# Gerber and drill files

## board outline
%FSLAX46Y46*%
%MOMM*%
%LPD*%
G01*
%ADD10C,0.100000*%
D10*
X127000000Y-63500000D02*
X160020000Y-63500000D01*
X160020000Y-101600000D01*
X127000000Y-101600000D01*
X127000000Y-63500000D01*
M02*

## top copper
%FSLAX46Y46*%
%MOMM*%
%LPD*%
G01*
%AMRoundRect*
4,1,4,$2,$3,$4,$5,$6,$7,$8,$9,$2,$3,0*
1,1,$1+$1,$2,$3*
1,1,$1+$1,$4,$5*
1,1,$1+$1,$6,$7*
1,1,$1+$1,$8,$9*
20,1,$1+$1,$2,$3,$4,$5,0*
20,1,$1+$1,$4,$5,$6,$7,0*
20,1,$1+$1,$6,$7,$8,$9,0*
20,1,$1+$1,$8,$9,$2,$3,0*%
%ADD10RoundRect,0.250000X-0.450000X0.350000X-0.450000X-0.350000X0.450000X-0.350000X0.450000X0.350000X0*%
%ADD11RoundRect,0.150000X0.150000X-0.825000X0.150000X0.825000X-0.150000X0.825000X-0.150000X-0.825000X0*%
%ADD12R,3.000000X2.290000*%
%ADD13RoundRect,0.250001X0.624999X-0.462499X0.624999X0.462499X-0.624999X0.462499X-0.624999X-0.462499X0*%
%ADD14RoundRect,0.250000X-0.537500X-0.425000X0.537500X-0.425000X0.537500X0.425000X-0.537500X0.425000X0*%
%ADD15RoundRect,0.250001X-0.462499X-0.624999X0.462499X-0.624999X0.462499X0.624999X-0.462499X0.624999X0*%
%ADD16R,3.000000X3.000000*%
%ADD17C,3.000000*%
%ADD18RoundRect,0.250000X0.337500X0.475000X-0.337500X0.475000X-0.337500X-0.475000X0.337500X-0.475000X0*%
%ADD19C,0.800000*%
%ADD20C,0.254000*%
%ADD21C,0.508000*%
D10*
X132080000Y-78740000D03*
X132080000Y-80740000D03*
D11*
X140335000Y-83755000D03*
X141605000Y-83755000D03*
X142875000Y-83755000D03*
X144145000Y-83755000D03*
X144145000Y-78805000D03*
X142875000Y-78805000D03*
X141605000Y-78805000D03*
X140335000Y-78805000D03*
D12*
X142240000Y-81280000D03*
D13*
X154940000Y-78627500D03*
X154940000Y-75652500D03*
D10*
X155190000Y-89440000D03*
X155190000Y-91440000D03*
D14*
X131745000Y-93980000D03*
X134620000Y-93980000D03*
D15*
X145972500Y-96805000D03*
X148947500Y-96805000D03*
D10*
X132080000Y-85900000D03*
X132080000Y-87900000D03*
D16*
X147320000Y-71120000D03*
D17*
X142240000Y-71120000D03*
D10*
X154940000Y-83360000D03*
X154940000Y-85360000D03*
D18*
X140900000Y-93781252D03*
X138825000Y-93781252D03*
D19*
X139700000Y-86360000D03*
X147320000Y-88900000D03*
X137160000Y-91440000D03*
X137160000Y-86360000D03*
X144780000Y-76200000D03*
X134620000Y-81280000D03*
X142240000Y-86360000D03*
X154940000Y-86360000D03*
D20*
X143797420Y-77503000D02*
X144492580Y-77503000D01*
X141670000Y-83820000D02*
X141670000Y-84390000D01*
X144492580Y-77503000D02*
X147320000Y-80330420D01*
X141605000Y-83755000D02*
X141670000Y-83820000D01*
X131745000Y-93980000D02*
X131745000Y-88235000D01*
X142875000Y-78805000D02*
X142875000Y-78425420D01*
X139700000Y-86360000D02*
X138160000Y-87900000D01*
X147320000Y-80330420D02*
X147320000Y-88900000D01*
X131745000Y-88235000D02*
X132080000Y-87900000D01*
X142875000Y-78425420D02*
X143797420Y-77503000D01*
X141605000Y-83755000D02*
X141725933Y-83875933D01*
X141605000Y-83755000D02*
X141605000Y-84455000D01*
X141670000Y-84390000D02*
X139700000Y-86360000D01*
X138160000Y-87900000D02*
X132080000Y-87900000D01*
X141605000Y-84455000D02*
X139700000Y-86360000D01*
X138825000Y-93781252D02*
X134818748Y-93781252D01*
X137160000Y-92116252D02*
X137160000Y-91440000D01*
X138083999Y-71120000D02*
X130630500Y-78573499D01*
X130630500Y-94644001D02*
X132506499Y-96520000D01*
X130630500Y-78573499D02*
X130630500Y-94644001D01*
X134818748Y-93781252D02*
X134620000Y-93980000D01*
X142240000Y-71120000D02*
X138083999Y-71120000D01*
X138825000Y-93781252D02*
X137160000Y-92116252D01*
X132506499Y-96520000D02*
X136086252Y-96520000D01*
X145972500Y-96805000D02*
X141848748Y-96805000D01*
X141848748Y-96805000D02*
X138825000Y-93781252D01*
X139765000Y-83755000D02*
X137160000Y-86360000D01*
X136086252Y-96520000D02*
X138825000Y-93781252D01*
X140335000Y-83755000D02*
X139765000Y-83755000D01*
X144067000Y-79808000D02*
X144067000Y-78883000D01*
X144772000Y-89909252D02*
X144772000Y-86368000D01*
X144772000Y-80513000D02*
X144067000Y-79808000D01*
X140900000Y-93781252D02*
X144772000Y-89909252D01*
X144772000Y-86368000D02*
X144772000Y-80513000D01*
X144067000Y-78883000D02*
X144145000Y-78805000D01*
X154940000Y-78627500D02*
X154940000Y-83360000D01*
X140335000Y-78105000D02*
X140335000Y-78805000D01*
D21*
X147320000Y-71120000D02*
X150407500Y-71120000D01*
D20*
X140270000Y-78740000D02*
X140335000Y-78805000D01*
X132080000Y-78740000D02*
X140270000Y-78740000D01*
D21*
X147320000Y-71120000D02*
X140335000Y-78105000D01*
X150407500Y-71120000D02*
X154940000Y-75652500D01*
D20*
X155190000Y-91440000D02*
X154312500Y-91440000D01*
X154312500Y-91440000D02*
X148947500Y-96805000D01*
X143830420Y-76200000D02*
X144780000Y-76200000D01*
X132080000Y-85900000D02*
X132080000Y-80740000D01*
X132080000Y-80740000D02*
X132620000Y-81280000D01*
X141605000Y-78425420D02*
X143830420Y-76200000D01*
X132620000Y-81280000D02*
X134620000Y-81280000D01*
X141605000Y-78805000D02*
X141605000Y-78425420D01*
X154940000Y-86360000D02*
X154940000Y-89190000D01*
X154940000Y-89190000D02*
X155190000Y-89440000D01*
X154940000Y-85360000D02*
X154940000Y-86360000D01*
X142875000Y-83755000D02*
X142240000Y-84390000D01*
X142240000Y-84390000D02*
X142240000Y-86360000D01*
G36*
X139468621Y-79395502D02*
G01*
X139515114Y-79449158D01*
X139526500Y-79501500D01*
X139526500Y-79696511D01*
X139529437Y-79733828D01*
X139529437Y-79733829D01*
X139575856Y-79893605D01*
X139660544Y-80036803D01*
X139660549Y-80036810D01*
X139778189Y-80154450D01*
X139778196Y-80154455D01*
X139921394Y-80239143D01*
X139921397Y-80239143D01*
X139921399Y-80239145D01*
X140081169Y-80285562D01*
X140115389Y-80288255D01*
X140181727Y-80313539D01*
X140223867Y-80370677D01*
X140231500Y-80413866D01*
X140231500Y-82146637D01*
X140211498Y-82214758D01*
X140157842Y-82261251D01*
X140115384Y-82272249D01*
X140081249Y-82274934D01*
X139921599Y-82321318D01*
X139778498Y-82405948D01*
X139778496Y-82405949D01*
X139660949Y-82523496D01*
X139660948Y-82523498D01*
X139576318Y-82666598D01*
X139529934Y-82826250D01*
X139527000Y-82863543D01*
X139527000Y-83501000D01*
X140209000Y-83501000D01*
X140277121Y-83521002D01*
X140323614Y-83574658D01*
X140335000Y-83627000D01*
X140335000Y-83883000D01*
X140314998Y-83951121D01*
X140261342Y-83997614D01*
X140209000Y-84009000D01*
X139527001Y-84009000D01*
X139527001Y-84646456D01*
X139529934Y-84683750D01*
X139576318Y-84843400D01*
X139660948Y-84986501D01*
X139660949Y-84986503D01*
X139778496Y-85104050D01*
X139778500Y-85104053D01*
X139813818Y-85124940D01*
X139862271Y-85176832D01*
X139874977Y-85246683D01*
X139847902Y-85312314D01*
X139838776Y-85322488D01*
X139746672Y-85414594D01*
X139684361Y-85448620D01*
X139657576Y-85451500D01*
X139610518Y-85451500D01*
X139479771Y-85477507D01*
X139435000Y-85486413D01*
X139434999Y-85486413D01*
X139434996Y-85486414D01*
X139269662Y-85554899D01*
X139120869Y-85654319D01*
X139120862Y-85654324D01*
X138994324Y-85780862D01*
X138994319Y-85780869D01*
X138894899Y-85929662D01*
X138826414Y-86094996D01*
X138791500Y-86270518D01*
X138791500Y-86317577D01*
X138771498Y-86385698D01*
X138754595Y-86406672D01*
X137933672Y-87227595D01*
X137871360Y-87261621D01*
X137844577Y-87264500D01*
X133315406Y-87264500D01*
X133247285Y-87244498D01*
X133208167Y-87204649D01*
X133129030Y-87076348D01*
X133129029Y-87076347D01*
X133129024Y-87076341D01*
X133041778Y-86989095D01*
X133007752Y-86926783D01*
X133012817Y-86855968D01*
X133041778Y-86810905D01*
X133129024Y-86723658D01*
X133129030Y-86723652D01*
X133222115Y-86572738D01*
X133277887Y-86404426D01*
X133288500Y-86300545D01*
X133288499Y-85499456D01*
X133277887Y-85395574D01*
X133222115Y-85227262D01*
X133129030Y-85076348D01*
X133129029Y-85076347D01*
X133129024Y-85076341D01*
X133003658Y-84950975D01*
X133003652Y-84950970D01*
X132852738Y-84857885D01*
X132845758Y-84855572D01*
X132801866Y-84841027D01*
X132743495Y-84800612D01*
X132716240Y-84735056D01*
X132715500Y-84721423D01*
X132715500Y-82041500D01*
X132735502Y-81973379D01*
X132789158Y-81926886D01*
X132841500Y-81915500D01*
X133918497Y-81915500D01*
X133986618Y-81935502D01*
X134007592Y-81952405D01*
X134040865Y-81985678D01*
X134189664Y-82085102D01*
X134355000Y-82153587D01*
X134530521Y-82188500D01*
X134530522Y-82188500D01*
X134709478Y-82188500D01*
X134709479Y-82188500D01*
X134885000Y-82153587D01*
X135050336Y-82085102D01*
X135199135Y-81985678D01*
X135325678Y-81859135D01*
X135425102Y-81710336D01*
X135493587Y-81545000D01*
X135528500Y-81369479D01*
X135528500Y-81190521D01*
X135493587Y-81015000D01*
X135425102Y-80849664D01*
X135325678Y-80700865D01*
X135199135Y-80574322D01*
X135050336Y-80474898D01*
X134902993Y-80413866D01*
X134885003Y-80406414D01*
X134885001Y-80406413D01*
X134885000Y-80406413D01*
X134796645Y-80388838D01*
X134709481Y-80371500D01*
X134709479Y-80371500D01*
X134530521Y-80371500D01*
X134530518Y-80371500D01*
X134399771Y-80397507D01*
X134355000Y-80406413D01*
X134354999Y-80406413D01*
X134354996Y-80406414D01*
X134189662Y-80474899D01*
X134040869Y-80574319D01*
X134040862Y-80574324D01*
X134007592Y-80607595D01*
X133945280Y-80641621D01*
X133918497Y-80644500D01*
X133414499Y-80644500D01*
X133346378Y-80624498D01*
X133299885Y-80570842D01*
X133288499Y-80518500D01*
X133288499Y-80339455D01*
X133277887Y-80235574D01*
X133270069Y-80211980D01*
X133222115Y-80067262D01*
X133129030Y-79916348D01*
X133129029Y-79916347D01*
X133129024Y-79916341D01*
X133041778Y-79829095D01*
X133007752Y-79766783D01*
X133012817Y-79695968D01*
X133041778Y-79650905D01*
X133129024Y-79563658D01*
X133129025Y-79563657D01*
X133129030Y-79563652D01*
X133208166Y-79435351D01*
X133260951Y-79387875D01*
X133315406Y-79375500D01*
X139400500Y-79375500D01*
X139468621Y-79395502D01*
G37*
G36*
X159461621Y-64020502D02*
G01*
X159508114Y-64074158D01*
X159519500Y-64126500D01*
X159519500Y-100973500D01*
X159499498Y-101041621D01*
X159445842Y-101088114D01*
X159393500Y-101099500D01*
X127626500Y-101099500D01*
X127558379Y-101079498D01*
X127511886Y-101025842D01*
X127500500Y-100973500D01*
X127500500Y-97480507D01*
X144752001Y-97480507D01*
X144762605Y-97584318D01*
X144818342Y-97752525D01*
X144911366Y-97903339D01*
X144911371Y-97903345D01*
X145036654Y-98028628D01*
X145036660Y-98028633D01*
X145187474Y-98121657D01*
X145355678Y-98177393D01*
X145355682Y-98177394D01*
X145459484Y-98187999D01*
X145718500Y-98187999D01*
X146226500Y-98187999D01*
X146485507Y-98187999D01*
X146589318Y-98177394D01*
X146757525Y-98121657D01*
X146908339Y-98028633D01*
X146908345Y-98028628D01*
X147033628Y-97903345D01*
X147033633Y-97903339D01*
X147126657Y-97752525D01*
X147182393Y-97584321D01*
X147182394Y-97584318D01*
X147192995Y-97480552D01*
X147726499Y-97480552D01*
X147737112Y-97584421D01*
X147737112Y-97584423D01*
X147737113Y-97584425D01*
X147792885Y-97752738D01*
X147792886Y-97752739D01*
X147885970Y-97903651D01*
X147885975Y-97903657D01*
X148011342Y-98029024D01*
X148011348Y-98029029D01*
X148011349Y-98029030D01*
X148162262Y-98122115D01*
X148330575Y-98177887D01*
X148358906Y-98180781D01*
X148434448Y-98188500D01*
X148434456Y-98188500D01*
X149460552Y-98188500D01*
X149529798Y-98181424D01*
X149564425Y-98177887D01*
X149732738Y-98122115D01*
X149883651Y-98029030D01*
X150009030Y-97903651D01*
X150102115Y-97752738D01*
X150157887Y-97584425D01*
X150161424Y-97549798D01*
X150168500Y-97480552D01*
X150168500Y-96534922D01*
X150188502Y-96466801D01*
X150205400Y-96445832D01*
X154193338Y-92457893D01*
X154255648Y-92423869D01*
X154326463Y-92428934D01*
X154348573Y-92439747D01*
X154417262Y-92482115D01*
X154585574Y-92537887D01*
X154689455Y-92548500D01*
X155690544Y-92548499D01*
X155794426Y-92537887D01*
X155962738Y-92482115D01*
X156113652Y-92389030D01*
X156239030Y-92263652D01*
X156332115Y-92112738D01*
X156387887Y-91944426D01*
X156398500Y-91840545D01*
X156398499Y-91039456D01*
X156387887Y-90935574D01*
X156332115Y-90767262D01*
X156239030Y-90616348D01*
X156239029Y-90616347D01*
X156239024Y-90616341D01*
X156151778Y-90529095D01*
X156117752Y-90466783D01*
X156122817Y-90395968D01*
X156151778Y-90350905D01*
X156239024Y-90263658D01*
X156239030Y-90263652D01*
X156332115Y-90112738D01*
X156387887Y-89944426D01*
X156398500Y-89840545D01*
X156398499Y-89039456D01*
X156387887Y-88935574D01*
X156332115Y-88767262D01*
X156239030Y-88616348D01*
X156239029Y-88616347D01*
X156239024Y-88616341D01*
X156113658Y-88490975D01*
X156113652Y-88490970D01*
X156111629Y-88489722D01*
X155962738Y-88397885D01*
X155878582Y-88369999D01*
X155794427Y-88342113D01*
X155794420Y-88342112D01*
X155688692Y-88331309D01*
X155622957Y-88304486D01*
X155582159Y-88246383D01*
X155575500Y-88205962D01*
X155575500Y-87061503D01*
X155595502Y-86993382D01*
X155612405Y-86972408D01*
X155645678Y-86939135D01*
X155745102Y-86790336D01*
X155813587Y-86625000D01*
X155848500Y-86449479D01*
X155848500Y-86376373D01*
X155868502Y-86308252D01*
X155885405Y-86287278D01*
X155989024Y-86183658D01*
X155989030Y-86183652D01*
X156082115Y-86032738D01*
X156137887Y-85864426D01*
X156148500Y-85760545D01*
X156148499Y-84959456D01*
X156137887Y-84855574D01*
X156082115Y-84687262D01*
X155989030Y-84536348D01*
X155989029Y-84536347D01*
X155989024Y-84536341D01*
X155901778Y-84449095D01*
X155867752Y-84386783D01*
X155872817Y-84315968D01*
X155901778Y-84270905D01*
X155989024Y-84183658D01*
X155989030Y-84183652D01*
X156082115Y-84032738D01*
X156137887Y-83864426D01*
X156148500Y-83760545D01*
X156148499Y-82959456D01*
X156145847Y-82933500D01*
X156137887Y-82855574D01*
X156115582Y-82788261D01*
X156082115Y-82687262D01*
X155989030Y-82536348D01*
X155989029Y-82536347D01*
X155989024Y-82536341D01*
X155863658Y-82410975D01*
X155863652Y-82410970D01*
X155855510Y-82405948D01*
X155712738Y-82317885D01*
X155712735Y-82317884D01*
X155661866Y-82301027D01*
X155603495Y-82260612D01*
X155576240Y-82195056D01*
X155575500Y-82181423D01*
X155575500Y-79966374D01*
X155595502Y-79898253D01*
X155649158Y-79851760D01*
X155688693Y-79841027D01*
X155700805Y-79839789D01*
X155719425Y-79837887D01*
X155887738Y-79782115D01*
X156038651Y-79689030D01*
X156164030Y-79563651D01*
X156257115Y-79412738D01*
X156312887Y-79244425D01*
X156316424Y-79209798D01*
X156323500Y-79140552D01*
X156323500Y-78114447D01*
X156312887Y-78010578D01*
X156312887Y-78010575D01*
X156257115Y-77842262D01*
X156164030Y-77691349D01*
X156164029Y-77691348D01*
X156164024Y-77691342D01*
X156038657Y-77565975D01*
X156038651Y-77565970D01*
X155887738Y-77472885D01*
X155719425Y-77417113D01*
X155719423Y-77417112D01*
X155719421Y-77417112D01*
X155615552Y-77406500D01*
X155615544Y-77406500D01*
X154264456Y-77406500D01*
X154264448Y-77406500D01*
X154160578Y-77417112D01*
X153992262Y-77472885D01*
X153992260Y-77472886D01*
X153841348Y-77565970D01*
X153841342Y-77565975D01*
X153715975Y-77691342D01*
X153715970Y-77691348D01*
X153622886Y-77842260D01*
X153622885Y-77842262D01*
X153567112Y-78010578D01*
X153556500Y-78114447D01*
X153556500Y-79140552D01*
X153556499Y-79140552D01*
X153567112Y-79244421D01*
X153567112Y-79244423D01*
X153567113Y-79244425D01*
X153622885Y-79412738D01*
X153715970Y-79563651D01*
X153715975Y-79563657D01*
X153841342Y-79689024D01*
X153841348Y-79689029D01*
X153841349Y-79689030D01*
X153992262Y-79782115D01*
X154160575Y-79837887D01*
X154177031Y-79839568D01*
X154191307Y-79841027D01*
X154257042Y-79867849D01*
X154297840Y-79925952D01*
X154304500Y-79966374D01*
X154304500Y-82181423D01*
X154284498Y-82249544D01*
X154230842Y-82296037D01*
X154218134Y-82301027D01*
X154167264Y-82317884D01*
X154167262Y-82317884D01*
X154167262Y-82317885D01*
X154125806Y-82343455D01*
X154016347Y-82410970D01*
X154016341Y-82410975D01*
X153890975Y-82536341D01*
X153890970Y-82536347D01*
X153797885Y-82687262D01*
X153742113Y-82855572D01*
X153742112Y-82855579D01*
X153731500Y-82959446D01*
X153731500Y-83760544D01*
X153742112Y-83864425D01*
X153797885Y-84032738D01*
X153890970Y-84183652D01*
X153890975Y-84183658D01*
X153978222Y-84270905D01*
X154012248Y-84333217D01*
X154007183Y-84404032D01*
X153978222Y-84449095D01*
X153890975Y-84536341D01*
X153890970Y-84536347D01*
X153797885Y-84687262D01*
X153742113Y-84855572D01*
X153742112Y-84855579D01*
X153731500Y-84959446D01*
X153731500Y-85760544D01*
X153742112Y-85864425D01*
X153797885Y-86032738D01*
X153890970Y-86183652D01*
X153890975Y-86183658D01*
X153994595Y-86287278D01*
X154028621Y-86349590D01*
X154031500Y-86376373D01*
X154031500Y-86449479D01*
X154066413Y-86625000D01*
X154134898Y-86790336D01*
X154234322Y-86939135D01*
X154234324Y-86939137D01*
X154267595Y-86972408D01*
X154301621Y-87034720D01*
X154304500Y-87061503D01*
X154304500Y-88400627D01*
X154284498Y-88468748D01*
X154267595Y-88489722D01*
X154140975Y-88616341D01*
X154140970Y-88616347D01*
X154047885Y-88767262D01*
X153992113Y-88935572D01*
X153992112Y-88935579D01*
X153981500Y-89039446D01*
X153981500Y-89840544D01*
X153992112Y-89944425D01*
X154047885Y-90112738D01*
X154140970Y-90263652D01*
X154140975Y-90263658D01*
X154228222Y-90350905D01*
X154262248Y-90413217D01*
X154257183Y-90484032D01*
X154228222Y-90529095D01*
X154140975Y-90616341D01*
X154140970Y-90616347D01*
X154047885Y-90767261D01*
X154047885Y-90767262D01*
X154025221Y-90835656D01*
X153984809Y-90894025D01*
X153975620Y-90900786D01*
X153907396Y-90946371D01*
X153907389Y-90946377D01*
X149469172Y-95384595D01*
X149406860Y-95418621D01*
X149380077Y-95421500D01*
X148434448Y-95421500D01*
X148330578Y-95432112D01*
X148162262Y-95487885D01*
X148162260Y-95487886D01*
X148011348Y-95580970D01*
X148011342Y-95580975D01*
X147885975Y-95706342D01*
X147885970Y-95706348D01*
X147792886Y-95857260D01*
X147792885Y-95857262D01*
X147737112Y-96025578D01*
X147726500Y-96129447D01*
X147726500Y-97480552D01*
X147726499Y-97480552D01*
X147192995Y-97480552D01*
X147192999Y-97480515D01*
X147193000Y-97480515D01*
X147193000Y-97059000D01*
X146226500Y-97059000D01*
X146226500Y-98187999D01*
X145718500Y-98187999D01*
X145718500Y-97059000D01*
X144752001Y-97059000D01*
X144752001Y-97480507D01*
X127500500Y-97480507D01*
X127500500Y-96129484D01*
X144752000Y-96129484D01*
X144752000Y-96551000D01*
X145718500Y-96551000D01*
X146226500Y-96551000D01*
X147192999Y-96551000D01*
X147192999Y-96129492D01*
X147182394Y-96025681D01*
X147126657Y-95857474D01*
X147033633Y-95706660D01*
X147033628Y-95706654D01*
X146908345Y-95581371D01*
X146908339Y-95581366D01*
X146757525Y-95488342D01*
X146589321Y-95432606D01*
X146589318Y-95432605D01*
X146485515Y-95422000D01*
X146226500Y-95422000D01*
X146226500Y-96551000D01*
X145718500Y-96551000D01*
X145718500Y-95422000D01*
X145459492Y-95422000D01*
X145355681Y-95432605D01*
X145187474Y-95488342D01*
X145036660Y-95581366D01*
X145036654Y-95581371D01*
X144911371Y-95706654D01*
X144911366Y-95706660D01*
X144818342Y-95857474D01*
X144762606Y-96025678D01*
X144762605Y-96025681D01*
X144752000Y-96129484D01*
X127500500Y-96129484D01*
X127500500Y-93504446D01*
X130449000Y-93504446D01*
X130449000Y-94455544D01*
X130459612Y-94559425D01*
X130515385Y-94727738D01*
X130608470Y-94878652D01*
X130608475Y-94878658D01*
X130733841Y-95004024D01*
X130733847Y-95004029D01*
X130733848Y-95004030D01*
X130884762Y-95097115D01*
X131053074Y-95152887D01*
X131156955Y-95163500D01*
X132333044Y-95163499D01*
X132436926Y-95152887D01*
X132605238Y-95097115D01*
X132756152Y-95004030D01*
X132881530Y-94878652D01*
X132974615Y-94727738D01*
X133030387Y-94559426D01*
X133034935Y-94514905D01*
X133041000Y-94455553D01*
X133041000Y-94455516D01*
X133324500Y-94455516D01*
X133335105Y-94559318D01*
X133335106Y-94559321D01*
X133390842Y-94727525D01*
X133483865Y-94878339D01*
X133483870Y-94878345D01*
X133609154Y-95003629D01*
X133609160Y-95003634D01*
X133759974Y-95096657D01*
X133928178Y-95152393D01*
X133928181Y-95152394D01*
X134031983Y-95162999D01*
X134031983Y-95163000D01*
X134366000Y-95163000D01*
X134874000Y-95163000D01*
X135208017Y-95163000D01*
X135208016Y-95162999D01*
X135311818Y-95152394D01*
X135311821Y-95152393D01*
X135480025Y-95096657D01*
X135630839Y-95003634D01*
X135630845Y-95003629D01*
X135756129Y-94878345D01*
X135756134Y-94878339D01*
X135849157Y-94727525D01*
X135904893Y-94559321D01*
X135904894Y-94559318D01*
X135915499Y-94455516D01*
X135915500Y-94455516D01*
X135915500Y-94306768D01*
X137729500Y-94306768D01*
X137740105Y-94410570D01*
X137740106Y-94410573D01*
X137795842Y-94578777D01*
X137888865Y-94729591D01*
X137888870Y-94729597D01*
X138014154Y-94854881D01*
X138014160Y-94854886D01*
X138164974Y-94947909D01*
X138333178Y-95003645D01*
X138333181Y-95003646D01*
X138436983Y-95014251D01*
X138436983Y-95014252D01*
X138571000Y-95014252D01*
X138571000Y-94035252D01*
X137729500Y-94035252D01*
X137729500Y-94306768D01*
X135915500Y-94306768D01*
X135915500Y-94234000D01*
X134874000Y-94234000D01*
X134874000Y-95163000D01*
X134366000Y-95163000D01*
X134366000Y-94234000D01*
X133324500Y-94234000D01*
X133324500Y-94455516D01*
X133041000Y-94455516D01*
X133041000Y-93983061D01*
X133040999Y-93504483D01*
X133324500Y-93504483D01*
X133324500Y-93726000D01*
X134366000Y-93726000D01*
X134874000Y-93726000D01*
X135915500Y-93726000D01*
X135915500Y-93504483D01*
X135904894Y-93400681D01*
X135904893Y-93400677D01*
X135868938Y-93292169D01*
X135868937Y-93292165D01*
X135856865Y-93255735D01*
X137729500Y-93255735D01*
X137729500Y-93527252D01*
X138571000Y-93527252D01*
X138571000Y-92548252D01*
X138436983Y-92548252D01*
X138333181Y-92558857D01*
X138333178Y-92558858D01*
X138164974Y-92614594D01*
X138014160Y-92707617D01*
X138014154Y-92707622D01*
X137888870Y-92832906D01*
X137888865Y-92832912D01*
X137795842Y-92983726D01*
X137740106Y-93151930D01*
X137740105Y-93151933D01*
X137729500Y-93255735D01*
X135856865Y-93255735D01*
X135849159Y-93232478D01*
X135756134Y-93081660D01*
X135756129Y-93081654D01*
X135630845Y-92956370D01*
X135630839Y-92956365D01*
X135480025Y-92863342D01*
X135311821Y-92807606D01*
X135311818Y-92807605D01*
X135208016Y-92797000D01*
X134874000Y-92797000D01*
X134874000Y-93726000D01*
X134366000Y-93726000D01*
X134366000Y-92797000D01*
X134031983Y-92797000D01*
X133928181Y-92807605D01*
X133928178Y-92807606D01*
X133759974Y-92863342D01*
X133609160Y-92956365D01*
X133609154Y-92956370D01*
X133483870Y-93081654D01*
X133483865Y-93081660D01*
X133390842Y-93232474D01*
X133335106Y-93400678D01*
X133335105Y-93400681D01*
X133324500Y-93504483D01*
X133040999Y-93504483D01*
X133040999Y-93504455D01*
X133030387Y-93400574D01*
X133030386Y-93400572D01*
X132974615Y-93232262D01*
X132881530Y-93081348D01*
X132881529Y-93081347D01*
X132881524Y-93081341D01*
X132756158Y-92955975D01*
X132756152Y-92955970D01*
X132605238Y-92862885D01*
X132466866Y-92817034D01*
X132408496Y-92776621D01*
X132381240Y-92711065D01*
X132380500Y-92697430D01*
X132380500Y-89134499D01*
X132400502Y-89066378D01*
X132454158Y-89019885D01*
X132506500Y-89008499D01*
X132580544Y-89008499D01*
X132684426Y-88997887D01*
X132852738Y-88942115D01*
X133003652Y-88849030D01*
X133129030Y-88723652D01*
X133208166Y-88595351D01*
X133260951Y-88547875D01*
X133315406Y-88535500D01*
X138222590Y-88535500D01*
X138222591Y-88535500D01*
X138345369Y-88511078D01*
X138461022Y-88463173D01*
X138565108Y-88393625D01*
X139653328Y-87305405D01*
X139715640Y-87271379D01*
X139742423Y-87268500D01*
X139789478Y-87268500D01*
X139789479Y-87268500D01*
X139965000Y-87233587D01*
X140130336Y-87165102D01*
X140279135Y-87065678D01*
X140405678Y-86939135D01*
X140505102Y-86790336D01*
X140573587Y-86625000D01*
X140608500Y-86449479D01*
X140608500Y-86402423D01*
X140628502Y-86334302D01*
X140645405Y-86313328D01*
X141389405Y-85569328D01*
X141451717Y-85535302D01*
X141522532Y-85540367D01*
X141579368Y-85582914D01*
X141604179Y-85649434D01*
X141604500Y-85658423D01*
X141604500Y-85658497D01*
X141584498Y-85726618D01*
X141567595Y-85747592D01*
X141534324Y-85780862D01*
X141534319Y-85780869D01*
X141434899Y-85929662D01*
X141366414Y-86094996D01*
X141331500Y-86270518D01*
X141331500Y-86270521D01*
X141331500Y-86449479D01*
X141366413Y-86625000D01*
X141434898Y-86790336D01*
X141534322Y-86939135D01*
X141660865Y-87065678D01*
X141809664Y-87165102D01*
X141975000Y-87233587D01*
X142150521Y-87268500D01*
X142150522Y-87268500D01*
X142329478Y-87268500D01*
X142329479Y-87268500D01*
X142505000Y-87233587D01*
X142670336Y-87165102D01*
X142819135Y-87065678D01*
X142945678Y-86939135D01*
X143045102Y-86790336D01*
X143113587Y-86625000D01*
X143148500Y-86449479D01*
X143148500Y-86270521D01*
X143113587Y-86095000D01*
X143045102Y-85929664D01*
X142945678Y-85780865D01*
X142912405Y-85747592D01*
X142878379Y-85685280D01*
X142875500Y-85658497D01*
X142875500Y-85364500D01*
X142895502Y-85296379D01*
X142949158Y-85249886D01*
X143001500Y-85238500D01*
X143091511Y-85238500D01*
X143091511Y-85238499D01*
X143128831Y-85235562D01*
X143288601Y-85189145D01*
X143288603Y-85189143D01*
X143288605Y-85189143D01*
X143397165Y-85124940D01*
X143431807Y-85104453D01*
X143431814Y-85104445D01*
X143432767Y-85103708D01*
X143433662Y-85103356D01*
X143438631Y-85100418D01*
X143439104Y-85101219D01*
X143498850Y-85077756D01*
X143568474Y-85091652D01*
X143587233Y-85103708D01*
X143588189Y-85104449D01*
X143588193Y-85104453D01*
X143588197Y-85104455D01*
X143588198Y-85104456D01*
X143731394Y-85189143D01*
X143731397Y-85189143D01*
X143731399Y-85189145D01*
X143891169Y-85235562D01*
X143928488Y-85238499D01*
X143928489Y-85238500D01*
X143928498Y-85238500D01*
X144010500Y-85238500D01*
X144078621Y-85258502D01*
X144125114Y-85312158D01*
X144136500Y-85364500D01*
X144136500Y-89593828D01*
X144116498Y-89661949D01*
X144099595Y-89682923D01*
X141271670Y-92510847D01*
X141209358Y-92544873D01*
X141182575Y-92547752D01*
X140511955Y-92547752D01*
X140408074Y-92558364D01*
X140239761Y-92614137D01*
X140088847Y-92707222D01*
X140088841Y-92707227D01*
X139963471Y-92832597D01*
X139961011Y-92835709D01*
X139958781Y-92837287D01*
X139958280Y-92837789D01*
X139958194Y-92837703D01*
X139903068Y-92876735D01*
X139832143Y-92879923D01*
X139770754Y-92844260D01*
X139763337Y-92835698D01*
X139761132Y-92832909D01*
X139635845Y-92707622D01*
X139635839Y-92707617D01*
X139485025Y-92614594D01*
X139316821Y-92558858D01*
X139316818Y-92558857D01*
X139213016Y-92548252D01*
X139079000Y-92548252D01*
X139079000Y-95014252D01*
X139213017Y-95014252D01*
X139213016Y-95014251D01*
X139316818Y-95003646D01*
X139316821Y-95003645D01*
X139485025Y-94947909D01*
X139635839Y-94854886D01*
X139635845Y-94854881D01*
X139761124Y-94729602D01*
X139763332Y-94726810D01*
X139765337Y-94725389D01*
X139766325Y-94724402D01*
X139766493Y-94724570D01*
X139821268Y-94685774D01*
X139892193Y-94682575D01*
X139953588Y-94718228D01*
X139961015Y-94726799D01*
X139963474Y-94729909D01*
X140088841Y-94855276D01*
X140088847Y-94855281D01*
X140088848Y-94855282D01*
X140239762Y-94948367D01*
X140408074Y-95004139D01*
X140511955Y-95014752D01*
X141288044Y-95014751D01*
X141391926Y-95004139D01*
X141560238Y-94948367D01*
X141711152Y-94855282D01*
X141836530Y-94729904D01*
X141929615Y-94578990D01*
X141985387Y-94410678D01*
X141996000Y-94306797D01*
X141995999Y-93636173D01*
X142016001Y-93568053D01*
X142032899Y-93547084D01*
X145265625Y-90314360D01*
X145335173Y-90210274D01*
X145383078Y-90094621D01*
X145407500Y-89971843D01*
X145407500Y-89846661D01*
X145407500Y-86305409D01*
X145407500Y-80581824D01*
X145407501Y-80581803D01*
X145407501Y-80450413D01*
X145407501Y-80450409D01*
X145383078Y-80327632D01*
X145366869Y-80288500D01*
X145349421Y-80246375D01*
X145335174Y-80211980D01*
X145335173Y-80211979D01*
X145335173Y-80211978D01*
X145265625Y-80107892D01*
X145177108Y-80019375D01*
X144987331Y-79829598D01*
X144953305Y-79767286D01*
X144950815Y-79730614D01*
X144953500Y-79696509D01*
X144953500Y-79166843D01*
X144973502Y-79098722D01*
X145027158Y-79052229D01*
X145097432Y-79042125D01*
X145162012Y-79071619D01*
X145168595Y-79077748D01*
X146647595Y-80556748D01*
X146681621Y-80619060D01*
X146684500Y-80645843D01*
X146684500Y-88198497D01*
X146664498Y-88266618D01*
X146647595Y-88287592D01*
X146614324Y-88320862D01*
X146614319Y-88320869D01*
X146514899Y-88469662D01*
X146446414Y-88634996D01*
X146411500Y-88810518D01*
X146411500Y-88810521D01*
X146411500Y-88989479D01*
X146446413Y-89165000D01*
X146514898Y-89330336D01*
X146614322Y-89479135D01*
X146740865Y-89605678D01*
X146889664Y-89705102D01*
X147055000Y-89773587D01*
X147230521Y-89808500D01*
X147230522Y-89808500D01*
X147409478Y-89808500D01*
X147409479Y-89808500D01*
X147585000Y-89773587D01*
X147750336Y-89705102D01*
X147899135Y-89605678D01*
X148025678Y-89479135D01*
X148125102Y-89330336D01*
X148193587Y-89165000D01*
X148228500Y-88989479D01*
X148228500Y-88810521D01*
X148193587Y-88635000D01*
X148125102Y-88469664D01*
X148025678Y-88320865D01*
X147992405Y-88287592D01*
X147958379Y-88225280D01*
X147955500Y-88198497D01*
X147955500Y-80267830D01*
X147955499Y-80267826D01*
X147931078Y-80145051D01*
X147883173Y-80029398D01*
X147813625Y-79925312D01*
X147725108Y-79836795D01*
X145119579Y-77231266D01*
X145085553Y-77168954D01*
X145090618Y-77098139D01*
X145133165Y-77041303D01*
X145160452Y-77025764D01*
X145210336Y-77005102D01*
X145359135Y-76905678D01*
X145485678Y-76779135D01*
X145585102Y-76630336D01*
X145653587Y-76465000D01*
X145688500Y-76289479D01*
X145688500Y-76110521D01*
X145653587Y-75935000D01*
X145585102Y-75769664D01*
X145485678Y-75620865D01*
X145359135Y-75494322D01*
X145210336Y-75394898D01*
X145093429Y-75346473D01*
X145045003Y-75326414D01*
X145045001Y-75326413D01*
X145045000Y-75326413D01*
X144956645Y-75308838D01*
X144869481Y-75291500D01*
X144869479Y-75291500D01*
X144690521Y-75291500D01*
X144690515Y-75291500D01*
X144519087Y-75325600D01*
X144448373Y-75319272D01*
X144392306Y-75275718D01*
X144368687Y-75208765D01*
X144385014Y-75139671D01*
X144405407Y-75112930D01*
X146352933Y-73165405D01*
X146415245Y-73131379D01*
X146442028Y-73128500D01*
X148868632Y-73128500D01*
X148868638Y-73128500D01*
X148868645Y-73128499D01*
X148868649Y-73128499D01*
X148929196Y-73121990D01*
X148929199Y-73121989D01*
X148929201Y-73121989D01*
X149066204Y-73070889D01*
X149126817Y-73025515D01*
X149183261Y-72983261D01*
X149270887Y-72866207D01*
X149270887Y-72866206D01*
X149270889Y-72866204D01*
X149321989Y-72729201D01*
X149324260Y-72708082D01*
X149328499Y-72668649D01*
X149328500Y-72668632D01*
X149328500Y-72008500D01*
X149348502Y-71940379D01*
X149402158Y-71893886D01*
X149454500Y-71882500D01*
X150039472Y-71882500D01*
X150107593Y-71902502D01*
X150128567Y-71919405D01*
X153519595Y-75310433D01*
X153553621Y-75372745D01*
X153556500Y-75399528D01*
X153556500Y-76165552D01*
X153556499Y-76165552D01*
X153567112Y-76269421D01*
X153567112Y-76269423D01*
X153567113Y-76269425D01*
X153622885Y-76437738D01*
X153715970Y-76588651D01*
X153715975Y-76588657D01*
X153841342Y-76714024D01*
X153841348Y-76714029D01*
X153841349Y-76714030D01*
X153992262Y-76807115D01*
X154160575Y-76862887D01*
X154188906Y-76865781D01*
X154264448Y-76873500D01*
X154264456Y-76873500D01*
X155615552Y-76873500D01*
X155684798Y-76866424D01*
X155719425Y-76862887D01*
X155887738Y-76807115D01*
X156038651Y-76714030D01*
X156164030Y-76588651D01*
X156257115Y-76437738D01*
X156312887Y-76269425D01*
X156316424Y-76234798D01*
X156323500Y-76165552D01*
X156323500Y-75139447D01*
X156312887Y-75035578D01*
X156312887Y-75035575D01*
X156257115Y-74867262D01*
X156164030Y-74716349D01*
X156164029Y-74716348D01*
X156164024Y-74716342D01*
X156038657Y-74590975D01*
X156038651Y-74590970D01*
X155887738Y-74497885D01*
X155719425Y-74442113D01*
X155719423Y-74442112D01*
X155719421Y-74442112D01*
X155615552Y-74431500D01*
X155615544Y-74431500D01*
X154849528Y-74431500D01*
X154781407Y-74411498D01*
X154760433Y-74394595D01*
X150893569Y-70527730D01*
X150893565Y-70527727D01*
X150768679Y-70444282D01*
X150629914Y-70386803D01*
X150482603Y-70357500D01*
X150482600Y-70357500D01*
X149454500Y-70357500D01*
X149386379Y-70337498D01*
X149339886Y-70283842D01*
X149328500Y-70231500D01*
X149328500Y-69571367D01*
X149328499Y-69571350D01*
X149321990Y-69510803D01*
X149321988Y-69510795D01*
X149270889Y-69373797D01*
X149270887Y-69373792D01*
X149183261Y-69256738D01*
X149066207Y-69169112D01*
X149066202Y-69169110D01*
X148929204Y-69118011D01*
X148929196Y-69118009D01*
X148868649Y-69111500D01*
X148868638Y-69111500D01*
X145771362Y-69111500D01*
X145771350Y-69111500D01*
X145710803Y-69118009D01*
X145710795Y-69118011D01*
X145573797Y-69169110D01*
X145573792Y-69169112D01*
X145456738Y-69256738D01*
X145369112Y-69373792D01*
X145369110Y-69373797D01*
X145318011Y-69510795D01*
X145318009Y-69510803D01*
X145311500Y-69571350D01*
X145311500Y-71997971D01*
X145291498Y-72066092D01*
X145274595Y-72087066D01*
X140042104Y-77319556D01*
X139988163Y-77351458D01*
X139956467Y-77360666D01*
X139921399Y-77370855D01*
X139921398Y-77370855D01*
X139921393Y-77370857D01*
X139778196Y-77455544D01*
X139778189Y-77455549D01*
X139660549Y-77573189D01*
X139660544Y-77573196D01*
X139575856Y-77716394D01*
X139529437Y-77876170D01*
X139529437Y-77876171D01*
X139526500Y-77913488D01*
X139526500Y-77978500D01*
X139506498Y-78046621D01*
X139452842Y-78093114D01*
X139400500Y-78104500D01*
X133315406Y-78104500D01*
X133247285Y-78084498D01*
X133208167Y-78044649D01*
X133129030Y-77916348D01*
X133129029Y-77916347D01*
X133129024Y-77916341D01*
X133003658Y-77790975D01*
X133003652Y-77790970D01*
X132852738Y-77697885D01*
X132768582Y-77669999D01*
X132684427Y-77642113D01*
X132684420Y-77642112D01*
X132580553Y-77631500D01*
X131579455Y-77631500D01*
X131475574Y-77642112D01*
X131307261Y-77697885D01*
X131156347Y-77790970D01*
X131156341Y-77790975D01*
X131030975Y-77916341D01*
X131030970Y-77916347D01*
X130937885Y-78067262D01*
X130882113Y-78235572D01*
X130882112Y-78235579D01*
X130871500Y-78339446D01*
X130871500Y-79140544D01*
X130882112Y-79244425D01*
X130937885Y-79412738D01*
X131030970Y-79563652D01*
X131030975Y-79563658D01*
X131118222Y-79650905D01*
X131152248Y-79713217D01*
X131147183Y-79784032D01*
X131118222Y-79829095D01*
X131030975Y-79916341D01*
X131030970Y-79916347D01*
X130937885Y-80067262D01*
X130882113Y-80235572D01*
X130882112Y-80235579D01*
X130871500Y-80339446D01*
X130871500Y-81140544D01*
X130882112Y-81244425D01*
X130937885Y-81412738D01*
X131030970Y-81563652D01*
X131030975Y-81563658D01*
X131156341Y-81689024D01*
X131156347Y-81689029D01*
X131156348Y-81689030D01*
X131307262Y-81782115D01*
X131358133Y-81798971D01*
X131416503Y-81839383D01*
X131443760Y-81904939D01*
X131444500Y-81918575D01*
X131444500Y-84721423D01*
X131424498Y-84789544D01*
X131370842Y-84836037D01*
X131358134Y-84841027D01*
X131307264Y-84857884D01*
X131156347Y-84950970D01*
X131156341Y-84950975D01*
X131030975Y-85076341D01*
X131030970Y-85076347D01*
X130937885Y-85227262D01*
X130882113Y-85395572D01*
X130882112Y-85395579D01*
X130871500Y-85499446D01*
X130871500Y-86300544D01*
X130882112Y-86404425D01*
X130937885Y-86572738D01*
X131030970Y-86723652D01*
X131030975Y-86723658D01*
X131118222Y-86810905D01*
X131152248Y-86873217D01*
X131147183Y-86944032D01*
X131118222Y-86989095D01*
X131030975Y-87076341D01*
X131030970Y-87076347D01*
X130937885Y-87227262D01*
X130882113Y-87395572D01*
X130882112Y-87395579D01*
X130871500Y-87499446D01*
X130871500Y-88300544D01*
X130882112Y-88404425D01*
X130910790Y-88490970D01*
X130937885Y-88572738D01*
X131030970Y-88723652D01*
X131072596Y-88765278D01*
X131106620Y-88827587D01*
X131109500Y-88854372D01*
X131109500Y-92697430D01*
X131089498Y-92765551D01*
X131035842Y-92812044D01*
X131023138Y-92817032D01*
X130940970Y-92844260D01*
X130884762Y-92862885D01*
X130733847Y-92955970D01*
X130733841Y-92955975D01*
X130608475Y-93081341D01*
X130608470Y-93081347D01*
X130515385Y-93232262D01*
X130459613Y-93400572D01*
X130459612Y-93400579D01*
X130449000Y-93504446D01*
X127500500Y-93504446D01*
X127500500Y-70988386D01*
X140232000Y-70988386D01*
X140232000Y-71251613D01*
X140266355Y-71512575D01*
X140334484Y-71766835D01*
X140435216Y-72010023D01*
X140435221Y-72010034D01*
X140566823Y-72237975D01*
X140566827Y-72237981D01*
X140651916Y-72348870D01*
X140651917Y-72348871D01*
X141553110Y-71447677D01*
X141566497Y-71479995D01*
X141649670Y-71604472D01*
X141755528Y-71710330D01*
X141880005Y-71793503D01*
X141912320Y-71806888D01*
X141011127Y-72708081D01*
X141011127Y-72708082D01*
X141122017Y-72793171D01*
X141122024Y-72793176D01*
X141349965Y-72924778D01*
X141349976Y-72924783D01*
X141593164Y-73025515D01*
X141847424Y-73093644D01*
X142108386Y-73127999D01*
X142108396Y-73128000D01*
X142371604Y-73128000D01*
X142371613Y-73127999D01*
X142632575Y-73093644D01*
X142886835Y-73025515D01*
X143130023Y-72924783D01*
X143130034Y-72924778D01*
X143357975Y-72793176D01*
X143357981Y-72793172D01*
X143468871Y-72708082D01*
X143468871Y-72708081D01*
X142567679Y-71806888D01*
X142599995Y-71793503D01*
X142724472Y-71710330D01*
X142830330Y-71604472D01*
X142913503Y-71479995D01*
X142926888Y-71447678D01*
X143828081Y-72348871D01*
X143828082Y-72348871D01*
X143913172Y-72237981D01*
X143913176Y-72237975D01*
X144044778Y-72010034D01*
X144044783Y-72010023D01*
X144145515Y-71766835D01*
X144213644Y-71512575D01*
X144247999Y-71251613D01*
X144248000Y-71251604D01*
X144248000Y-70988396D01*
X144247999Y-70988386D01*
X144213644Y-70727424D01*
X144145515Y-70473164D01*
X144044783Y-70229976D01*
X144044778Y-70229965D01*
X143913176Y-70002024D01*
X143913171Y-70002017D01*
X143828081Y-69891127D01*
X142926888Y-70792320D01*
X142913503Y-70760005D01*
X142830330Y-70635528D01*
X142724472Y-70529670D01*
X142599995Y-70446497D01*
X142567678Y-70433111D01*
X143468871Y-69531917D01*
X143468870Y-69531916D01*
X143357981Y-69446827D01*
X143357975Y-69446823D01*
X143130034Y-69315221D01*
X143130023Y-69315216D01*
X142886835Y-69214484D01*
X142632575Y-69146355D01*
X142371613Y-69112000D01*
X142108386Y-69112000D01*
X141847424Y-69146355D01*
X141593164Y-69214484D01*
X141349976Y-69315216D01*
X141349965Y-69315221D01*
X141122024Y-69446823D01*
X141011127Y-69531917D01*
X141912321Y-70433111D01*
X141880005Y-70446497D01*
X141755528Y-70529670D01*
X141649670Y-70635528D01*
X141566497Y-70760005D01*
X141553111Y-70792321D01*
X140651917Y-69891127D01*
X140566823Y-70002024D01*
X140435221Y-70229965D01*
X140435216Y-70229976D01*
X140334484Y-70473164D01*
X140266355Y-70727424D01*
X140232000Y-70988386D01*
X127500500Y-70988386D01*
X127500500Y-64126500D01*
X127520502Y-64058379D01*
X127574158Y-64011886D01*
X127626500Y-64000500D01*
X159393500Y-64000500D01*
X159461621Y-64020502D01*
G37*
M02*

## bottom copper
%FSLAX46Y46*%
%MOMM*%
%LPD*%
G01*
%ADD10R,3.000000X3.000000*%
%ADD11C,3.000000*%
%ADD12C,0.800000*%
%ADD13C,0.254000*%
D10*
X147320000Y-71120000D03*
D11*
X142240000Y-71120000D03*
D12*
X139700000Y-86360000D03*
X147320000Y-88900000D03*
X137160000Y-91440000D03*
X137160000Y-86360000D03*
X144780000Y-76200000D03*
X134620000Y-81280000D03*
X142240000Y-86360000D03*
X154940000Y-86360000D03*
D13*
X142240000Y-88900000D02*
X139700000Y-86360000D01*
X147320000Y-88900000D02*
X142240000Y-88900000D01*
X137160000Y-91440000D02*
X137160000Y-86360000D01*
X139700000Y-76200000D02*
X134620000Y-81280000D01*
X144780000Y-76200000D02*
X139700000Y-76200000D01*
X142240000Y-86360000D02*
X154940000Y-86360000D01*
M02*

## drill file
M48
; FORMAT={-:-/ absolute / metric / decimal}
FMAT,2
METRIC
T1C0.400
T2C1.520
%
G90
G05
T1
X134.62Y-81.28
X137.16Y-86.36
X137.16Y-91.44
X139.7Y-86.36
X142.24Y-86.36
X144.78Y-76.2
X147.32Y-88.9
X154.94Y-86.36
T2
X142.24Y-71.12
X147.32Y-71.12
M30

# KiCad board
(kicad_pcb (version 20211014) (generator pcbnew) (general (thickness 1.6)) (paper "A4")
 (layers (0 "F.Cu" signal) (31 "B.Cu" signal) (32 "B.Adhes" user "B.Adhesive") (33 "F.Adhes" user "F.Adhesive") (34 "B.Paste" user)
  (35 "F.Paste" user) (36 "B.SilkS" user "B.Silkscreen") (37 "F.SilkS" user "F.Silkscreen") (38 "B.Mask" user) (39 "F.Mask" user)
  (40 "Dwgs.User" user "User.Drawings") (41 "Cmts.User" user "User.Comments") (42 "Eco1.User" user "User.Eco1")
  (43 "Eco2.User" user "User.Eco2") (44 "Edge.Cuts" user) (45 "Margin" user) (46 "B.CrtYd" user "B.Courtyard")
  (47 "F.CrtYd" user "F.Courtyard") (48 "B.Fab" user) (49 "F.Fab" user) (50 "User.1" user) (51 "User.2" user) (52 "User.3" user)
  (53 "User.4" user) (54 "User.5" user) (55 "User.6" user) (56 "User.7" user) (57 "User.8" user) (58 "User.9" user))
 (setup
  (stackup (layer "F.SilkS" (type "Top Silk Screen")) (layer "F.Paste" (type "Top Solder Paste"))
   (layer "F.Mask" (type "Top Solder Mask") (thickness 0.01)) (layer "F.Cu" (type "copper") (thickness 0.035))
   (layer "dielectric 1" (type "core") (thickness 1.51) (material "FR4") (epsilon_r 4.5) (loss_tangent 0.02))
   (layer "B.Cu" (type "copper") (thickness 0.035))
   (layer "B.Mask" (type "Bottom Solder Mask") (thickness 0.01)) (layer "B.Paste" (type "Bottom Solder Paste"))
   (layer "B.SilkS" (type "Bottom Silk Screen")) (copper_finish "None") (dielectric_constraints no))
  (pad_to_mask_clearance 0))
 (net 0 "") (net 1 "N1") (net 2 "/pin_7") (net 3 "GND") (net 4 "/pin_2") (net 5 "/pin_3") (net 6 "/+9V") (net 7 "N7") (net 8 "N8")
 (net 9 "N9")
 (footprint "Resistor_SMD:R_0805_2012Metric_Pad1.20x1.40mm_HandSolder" (layer "F.Cu") (at 132.08 79.74 -90)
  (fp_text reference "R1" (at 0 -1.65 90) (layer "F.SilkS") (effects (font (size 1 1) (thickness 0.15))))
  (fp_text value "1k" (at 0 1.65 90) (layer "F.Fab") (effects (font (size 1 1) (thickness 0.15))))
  (pad "1" smd roundrect (at -1 0 270) (size 1.2 1.4) (layers "F.Cu" "F.Paste" "F.Mask") (roundrect_rratio 0.2083333333) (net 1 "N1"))
  (pad "2" smd roundrect (at 1 0 270) (size 1.2 1.4) (layers "F.Cu" "F.Paste" "F.Mask") (roundrect_rratio 0.2083333333) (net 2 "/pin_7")))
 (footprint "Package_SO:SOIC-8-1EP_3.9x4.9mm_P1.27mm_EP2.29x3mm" (layer "F.Cu") (at 142.24 81.28 90)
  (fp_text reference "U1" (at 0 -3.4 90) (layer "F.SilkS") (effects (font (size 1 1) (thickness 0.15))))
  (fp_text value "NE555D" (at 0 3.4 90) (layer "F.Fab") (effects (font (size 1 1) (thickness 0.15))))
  (pad "" smd roundrect (at 0.57 0.75 90) (size 0.92 1.21) (layers "F.Paste") (roundrect_rratio 0.25))
  (pad "" smd roundrect (at -0.57 -0.75 90) (size 0.92 1.21) (layers "F.Paste") (roundrect_rratio 0.25))
  (pad "" smd roundrect (at 0.57 -0.75 90) (size 0.92 1.21) (layers "F.Paste") (roundrect_rratio 0.25))
  (pad "" smd roundrect (at -0.57 0.75 90) (size 0.92 1.21) (layers "F.Paste") (roundrect_rratio 0.25))
  (pad "1" smd roundrect (at -2.475 -1.905 90) (size 1.95 0.6) (layers "F.Cu" "F.Paste" "F.Mask") (roundrect_rratio 0.25) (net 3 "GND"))
  (pad "2" smd roundrect (at -2.475 -0.635 90) (size 1.95 0.6) (layers "F.Cu" "F.Paste" "F.Mask") (roundrect_rratio 0.25) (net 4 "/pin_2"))
  (pad "3" smd roundrect (at -2.475 0.635 90) (size 1.95 0.6) (layers "F.Cu" "F.Paste" "F.Mask") (roundrect_rratio 0.25) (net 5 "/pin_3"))
  (pad "4" smd roundrect (at -2.475 1.905 90) (size 1.95 0.6) (layers "F.Cu" "F.Paste" "F.Mask") (roundrect_rratio 0.25) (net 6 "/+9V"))
  (pad "5" smd roundrect (at 2.475 1.905 90) (size 1.95 0.6) (layers "F.Cu" "F.Paste" "F.Mask") (roundrect_rratio 0.25) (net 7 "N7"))
  (pad "6" smd roundrect (at 2.475 0.635 90) (size 1.95 0.6) (layers "F.Cu" "F.Paste" "F.Mask") (roundrect_rratio 0.25) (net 4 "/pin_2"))
  (pad "7" smd roundrect (at 2.475 -0.635 90) (size 1.95 0.6) (layers "F.Cu" "F.Paste" "F.Mask") (roundrect_rratio 0.25) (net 2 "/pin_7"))
  (pad "8" smd roundrect (at 2.475 -1.905 90) (size 1.95 0.6) (layers "F.Cu" "F.Paste" "F.Mask") (roundrect_rratio 0.25) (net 1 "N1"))
  (pad "9" smd rect (at 0 0 90) (size 2.29 3) (layers "F.Cu" "F.Mask")))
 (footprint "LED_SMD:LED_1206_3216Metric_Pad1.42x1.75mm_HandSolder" (layer "F.Cu") (at 154.94 77.14 90)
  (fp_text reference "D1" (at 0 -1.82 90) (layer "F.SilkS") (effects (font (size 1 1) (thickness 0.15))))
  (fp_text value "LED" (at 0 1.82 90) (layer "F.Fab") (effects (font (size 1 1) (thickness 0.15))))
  (pad "1" smd roundrect (at -1.4875 0 90) (size 1.425 1.75) (layers "F.Cu" "F.Paste" "F.Mask") (roundrect_rratio 0.1754392982) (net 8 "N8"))
  (pad "2" smd roundrect (at 1.4875 0 90) (size 1.425 1.75) (layers "F.Cu" "F.Paste" "F.Mask") (roundrect_rratio 0.1754392982) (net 1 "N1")))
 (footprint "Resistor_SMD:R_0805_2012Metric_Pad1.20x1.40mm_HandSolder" (layer "F.Cu") (at 155.19 90.44 -90)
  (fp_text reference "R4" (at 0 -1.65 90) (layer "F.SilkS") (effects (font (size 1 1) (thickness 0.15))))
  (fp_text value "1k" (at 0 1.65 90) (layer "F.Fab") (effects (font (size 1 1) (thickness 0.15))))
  (pad "1" smd roundrect (at -1 0 270) (size 1.2 1.4) (layers "F.Cu" "F.Paste" "F.Mask") (roundrect_rratio 0.2083333333) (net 5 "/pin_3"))
  (pad "2" smd roundrect (at 1 0 270) (size 1.2 1.4) (layers "F.Cu" "F.Paste" "F.Mask") (roundrect_rratio 0.2083333333) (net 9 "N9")))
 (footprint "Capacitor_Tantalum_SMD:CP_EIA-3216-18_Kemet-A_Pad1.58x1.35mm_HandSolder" (layer "F.Cu") (at 133.1825 93.98)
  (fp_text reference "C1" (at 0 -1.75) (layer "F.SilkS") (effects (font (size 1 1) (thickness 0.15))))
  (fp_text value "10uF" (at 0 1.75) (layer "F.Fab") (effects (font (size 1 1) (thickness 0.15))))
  (pad "1" smd roundrect (at -1.4375 0) (size 1.575 1.35) (layers "F.Cu" "F.Paste" "F.Mask") (roundrect_rratio 0.1851851852)
   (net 4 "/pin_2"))
  (pad "2" smd roundrect (at 1.4375 0) (size 1.575 1.35) (layers "F.Cu" "F.Paste" "F.Mask") (roundrect_rratio 0.1851851852) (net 3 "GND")))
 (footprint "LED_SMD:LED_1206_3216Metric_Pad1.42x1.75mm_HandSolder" (layer "F.Cu") (at 147.46 96.805)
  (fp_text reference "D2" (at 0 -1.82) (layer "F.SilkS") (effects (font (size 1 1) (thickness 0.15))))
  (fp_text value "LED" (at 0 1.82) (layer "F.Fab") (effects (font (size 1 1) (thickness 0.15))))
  (pad "1" smd roundrect (at -1.4875 0) (size 1.425 1.75) (layers "F.Cu" "F.Paste" "F.Mask") (roundrect_rratio 0.1754392982) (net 3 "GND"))
  (pad "2" smd roundrect (at 1.4875 0) (size 1.425 1.75) (layers "F.Cu" "F.Paste" "F.Mask") (roundrect_rratio 0.1754392982) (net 9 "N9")))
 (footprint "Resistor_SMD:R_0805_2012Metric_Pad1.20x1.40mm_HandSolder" (layer "F.Cu") (at 132.08 86.9 -90)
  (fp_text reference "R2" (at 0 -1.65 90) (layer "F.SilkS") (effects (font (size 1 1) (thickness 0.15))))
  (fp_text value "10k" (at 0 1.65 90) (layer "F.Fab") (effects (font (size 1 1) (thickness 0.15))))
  (pad "1" smd roundrect (at -1 0 270) (size 1.2 1.4) (layers "F.Cu" "F.Paste" "F.Mask") (roundrect_rratio 0.2083333333) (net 2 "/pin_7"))
  (pad "2" smd roundrect (at 1 0 270) (size 1.2 1.4) (layers "F.Cu" "F.Paste" "F.Mask") (roundrect_rratio 0.2083333333) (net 4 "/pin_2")))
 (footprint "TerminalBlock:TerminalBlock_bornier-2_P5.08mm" (layer "F.Cu") (at 147.32 71.12 180)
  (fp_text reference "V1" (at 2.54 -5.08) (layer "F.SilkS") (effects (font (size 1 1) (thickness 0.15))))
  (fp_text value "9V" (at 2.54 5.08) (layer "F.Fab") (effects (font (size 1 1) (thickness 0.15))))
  (pad "1" thru_hole rect (at 0 0 180) (size 3 3) (drill 1.52) (layers *.Cu *.Mask) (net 1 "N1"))
  (pad "2" thru_hole circle (at 5.08 0 180) (size 3 3) (drill 1.52) (layers *.Cu *.Mask) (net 3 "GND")))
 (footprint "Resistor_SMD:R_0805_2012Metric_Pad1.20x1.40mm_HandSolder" (layer "F.Cu") (at 154.94 84.36 -90)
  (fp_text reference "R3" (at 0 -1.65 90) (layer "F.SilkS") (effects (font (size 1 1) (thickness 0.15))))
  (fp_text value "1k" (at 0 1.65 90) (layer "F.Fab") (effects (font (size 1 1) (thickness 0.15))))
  (pad "1" smd roundrect (at -1 0 270) (size 1.2 1.4) (layers "F.Cu" "F.Paste" "F.Mask") (roundrect_rratio 0.2083333333) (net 8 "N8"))
  (pad "2" smd roundrect (at 1 0 270) (size 1.2 1.4) (layers "F.Cu" "F.Paste" "F.Mask") (roundrect_rratio 0.2083333333) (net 5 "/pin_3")))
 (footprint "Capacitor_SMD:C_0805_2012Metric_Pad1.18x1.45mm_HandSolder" (layer "F.Cu") (at 139.8625 93.781252 180)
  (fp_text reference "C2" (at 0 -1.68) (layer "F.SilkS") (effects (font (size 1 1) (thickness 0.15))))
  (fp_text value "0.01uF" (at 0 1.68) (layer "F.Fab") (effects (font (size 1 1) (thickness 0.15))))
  (pad "1" smd roundrect (at -1.0375 0 180) (size 1.175 1.45) (layers "F.Cu" "F.Paste" "F.Mask") (roundrect_rratio 0.2127659574)
   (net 7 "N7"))
  (pad "2" smd roundrect (at 1.0375 0 180) (size 1.175 1.45) (layers "F.Cu" "F.Paste" "F.Mask") (roundrect_rratio 0.2127659574)
   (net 3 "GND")))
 (gr_rect (start 127 63.5) (end 160.02 101.6) (layer "Edge.Cuts") (width 0.1) (fill none))
 (segment (start 143.79742 77.503) (end 144.49258 77.503) (width 0.254) (layer "F.Cu") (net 4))
 (segment (start 141.67 83.82) (end 141.67 84.39) (width 0.254) (layer "F.Cu") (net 4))
 (segment (start 144.49258 77.503) (end 147.32 80.33042) (width 0.254) (layer "F.Cu") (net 4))
 (segment (start 141.605 83.755) (end 141.67 83.82) (width 0.254) (layer "F.Cu") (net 4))
 (segment (start 131.745 93.98) (end 131.745 88.235) (width 0.254) (layer "F.Cu") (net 4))
 (segment (start 142.875 78.805) (end 142.875 78.42542) (width 0.254) (layer "F.Cu") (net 4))
 (segment (start 139.7 86.36) (end 138.16 87.9) (width 0.254) (layer "F.Cu") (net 4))
 (segment (start 147.32 80.33042) (end 147.32 88.9) (width 0.254) (layer "F.Cu") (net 4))
 (segment (start 131.745 88.235) (end 132.08 87.9) (width 0.254) (layer "F.Cu") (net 4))
 (segment (start 142.875 78.42542) (end 143.79742 77.503) (width 0.254) (layer "F.Cu") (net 4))
 (segment (start 141.605 83.755) (end 141.725933 83.875933) (width 0.254) (layer "F.Cu") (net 4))
 (segment (start 141.605 83.755) (end 141.605 84.455) (width 0.254) (layer "F.Cu") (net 4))
 (segment (start 141.67 84.39) (end 139.7 86.36) (width 0.254) (layer "F.Cu") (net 4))
 (segment (start 138.16 87.9) (end 132.08 87.9) (width 0.254) (layer "F.Cu") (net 4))
 (segment (start 141.605 84.455) (end 139.7 86.36) (width 0.254) (layer "F.Cu") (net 4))
 (via (at 139.7 86.36) (size 0.8) (drill 0.4) (layers "F.Cu" "B.Cu") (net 4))
 (via (at 147.32 88.9) (size 0.8) (drill 0.4) (layers "F.Cu" "B.Cu") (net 4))
 (segment (start 142.24 88.9) (end 139.7 86.36) (width 0.254) (layer "B.Cu") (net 4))
 (segment (start 147.32 88.9) (end 142.24 88.9) (width 0.254) (layer "B.Cu") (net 4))
 (segment (start 138.825 93.781252) (end 134.818748 93.781252) (width 0.254) (layer "F.Cu") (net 3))
 (segment (start 137.16 92.116252) (end 137.16 91.44) (width 0.254) (layer "F.Cu") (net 3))
 (segment (start 138.083999 71.12) (end 130.6305 78.573499) (width 0.254) (layer "F.Cu") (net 3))
 (segment (start 130.6305 94.644001) (end 132.506499 96.52) (width 0.254) (layer "F.Cu") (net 3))
 (segment (start 130.6305 78.573499) (end 130.6305 94.644001) (width 0.254) (layer "F.Cu") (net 3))
 (segment (start 134.818748 93.781252) (end 134.62 93.98) (width 0.254) (layer "F.Cu") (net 3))
 (segment (start 142.24 71.12) (end 138.083999 71.12) (width 0.254) (layer "F.Cu") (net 3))
 (segment (start 138.825 93.781252) (end 137.16 92.116252) (width 0.254) (layer "F.Cu") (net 3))
 (segment (start 132.506499 96.52) (end 136.086252 96.52) (width 0.254) (layer "F.Cu") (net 3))
 (segment (start 145.9725 96.805) (end 141.848748 96.805) (width 0.254) (layer "F.Cu") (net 3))
 (segment (start 141.848748 96.805) (end 138.825 93.781252) (width 0.254) (layer "F.Cu") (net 3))
 (segment (start 139.765 83.755) (end 137.16 86.36) (width 0.254) (layer "F.Cu") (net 3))
 (segment (start 136.086252 96.52) (end 138.825 93.781252) (width 0.254) (layer "F.Cu") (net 3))
 (segment (start 140.335 83.755) (end 139.765 83.755) (width 0.254) (layer "F.Cu") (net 3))
 (via (at 137.16 91.44) (size 0.8) (drill 0.4) (layers "F.Cu" "B.Cu") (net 3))
 (via (at 137.16 86.36) (size 0.8) (drill 0.4) (layers "F.Cu" "B.Cu") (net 3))
 (segment (start 137.16 91.44) (end 137.16 86.36) (width 0.254) (layer "B.Cu") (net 3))
 (segment (start 144.067 79.808) (end 144.067 78.883) (width 0.254) (layer "F.Cu") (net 7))
 (segment (start 144.772 89.909252) (end 144.772 86.368) (width 0.254) (layer "F.Cu") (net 7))
 (segment (start 144.772 80.513) (end 144.067 79.808) (width 0.254) (layer "F.Cu") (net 7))
 (segment (start 140.9 93.781252) (end 144.772 89.909252) (width 0.254) (layer "F.Cu") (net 7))
 (segment (start 144.772 86.368) (end 144.772 80.513) (width 0.254) (layer "F.Cu") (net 7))
 (segment (start 144.067 78.883) (end 144.145 78.805) (width 0.254) (layer "F.Cu") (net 7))
 (segment (start 154.94 78.6275) (end 154.94 83.36) (width 0.254) (layer "F.Cu") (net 8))
 (segment (start 140.335 78.105) (end 140.335 78.805) (width 0.254) (layer "F.Cu") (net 1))
 (segment (start 147.32 71.12) (end 150.4075 71.12) (width 0.508) (layer "F.Cu") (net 1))
 (segment (start 140.27 78.74) (end 140.335 78.805) (width 0.254) (layer "F.Cu") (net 1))
 (segment (start 132.08 78.74) (end 140.27 78.74) (width 0.254) (layer "F.Cu") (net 1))
 (segment (start 147.32 71.12) (end 140.335 78.105) (width 0.508) (layer "F.Cu") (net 1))
 (segment (start 150.4075 71.12) (end 154.94 75.6525) (width 0.508) (layer "F.Cu") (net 1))
 (segment (start 155.19 91.44) (end 154.3125 91.44) (width 0.254) (layer "F.Cu") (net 9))
 (segment (start 154.3125 91.44) (end 148.9475 96.805) (width 0.254) (layer "F.Cu") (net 9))
 (segment (start 143.83042 76.2) (end 144.78 76.2) (width 0.254) (layer "F.Cu") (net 2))
 (segment (start 132.08 85.9) (end 132.08 80.74) (width 0.254) (layer "F.Cu") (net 2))
 (segment (start 132.08 80.74) (end 132.62 81.28) (width 0.254) (layer "F.Cu") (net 2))
 (segment (start 141.605 78.42542) (end 143.83042 76.2) (width 0.254) (layer "F.Cu") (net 2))
 (segment (start 132.62 81.28) (end 134.62 81.28) (width 0.254) (layer "F.Cu") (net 2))
 (segment (start 141.605 78.805) (end 141.605 78.42542) (width 0.254) (layer "F.Cu") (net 2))
 (via (at 144.78 76.2) (size 0.8) (drill 0.4) (layers "F.Cu" "B.Cu") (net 2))
 (via (at 134.62 81.28) (size 0.8) (drill 0.4) (layers "F.Cu" "B.Cu") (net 2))
 (segment (start 139.7 76.2) (end 134.62 81.28) (width 0.254) (layer "B.Cu") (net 2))
 (segment (start 144.78 76.2) (end 139.7 76.2) (width 0.254) (layer "B.Cu") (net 2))
 (segment (start 154.94 86.36) (end 154.94 89.19) (width 0.254) (layer "F.Cu") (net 5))
 (segment (start 154.94 89.19) (end 155.19 89.44) (width 0.254) (layer "F.Cu") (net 5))
 (segment (start 154.94 85.36) (end 154.94 86.36) (width 0.254) (layer "F.Cu") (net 5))
 (segment (start 142.875 83.755) (end 142.24 84.39) (width 0.254) (layer "F.Cu") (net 5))
 (segment (start 142.24 84.39) (end 142.24 86.36) (width 0.254) (layer "F.Cu") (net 5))
 (via (at 142.24 86.36) (size 0.8) (drill 0.4) (layers "F.Cu" "B.Cu") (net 5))
 (via (at 154.94 86.36) (size 0.8) (drill 0.4) (layers "F.Cu" "B.Cu") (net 5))
 (segment (start 142.24 86.36) (end 154.94 86.36) (width 0.254) (layer "B.Cu") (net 5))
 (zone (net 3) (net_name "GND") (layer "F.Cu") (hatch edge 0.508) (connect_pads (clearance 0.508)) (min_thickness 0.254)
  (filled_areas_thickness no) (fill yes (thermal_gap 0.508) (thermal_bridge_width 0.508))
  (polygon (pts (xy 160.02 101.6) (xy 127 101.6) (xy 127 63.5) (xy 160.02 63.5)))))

